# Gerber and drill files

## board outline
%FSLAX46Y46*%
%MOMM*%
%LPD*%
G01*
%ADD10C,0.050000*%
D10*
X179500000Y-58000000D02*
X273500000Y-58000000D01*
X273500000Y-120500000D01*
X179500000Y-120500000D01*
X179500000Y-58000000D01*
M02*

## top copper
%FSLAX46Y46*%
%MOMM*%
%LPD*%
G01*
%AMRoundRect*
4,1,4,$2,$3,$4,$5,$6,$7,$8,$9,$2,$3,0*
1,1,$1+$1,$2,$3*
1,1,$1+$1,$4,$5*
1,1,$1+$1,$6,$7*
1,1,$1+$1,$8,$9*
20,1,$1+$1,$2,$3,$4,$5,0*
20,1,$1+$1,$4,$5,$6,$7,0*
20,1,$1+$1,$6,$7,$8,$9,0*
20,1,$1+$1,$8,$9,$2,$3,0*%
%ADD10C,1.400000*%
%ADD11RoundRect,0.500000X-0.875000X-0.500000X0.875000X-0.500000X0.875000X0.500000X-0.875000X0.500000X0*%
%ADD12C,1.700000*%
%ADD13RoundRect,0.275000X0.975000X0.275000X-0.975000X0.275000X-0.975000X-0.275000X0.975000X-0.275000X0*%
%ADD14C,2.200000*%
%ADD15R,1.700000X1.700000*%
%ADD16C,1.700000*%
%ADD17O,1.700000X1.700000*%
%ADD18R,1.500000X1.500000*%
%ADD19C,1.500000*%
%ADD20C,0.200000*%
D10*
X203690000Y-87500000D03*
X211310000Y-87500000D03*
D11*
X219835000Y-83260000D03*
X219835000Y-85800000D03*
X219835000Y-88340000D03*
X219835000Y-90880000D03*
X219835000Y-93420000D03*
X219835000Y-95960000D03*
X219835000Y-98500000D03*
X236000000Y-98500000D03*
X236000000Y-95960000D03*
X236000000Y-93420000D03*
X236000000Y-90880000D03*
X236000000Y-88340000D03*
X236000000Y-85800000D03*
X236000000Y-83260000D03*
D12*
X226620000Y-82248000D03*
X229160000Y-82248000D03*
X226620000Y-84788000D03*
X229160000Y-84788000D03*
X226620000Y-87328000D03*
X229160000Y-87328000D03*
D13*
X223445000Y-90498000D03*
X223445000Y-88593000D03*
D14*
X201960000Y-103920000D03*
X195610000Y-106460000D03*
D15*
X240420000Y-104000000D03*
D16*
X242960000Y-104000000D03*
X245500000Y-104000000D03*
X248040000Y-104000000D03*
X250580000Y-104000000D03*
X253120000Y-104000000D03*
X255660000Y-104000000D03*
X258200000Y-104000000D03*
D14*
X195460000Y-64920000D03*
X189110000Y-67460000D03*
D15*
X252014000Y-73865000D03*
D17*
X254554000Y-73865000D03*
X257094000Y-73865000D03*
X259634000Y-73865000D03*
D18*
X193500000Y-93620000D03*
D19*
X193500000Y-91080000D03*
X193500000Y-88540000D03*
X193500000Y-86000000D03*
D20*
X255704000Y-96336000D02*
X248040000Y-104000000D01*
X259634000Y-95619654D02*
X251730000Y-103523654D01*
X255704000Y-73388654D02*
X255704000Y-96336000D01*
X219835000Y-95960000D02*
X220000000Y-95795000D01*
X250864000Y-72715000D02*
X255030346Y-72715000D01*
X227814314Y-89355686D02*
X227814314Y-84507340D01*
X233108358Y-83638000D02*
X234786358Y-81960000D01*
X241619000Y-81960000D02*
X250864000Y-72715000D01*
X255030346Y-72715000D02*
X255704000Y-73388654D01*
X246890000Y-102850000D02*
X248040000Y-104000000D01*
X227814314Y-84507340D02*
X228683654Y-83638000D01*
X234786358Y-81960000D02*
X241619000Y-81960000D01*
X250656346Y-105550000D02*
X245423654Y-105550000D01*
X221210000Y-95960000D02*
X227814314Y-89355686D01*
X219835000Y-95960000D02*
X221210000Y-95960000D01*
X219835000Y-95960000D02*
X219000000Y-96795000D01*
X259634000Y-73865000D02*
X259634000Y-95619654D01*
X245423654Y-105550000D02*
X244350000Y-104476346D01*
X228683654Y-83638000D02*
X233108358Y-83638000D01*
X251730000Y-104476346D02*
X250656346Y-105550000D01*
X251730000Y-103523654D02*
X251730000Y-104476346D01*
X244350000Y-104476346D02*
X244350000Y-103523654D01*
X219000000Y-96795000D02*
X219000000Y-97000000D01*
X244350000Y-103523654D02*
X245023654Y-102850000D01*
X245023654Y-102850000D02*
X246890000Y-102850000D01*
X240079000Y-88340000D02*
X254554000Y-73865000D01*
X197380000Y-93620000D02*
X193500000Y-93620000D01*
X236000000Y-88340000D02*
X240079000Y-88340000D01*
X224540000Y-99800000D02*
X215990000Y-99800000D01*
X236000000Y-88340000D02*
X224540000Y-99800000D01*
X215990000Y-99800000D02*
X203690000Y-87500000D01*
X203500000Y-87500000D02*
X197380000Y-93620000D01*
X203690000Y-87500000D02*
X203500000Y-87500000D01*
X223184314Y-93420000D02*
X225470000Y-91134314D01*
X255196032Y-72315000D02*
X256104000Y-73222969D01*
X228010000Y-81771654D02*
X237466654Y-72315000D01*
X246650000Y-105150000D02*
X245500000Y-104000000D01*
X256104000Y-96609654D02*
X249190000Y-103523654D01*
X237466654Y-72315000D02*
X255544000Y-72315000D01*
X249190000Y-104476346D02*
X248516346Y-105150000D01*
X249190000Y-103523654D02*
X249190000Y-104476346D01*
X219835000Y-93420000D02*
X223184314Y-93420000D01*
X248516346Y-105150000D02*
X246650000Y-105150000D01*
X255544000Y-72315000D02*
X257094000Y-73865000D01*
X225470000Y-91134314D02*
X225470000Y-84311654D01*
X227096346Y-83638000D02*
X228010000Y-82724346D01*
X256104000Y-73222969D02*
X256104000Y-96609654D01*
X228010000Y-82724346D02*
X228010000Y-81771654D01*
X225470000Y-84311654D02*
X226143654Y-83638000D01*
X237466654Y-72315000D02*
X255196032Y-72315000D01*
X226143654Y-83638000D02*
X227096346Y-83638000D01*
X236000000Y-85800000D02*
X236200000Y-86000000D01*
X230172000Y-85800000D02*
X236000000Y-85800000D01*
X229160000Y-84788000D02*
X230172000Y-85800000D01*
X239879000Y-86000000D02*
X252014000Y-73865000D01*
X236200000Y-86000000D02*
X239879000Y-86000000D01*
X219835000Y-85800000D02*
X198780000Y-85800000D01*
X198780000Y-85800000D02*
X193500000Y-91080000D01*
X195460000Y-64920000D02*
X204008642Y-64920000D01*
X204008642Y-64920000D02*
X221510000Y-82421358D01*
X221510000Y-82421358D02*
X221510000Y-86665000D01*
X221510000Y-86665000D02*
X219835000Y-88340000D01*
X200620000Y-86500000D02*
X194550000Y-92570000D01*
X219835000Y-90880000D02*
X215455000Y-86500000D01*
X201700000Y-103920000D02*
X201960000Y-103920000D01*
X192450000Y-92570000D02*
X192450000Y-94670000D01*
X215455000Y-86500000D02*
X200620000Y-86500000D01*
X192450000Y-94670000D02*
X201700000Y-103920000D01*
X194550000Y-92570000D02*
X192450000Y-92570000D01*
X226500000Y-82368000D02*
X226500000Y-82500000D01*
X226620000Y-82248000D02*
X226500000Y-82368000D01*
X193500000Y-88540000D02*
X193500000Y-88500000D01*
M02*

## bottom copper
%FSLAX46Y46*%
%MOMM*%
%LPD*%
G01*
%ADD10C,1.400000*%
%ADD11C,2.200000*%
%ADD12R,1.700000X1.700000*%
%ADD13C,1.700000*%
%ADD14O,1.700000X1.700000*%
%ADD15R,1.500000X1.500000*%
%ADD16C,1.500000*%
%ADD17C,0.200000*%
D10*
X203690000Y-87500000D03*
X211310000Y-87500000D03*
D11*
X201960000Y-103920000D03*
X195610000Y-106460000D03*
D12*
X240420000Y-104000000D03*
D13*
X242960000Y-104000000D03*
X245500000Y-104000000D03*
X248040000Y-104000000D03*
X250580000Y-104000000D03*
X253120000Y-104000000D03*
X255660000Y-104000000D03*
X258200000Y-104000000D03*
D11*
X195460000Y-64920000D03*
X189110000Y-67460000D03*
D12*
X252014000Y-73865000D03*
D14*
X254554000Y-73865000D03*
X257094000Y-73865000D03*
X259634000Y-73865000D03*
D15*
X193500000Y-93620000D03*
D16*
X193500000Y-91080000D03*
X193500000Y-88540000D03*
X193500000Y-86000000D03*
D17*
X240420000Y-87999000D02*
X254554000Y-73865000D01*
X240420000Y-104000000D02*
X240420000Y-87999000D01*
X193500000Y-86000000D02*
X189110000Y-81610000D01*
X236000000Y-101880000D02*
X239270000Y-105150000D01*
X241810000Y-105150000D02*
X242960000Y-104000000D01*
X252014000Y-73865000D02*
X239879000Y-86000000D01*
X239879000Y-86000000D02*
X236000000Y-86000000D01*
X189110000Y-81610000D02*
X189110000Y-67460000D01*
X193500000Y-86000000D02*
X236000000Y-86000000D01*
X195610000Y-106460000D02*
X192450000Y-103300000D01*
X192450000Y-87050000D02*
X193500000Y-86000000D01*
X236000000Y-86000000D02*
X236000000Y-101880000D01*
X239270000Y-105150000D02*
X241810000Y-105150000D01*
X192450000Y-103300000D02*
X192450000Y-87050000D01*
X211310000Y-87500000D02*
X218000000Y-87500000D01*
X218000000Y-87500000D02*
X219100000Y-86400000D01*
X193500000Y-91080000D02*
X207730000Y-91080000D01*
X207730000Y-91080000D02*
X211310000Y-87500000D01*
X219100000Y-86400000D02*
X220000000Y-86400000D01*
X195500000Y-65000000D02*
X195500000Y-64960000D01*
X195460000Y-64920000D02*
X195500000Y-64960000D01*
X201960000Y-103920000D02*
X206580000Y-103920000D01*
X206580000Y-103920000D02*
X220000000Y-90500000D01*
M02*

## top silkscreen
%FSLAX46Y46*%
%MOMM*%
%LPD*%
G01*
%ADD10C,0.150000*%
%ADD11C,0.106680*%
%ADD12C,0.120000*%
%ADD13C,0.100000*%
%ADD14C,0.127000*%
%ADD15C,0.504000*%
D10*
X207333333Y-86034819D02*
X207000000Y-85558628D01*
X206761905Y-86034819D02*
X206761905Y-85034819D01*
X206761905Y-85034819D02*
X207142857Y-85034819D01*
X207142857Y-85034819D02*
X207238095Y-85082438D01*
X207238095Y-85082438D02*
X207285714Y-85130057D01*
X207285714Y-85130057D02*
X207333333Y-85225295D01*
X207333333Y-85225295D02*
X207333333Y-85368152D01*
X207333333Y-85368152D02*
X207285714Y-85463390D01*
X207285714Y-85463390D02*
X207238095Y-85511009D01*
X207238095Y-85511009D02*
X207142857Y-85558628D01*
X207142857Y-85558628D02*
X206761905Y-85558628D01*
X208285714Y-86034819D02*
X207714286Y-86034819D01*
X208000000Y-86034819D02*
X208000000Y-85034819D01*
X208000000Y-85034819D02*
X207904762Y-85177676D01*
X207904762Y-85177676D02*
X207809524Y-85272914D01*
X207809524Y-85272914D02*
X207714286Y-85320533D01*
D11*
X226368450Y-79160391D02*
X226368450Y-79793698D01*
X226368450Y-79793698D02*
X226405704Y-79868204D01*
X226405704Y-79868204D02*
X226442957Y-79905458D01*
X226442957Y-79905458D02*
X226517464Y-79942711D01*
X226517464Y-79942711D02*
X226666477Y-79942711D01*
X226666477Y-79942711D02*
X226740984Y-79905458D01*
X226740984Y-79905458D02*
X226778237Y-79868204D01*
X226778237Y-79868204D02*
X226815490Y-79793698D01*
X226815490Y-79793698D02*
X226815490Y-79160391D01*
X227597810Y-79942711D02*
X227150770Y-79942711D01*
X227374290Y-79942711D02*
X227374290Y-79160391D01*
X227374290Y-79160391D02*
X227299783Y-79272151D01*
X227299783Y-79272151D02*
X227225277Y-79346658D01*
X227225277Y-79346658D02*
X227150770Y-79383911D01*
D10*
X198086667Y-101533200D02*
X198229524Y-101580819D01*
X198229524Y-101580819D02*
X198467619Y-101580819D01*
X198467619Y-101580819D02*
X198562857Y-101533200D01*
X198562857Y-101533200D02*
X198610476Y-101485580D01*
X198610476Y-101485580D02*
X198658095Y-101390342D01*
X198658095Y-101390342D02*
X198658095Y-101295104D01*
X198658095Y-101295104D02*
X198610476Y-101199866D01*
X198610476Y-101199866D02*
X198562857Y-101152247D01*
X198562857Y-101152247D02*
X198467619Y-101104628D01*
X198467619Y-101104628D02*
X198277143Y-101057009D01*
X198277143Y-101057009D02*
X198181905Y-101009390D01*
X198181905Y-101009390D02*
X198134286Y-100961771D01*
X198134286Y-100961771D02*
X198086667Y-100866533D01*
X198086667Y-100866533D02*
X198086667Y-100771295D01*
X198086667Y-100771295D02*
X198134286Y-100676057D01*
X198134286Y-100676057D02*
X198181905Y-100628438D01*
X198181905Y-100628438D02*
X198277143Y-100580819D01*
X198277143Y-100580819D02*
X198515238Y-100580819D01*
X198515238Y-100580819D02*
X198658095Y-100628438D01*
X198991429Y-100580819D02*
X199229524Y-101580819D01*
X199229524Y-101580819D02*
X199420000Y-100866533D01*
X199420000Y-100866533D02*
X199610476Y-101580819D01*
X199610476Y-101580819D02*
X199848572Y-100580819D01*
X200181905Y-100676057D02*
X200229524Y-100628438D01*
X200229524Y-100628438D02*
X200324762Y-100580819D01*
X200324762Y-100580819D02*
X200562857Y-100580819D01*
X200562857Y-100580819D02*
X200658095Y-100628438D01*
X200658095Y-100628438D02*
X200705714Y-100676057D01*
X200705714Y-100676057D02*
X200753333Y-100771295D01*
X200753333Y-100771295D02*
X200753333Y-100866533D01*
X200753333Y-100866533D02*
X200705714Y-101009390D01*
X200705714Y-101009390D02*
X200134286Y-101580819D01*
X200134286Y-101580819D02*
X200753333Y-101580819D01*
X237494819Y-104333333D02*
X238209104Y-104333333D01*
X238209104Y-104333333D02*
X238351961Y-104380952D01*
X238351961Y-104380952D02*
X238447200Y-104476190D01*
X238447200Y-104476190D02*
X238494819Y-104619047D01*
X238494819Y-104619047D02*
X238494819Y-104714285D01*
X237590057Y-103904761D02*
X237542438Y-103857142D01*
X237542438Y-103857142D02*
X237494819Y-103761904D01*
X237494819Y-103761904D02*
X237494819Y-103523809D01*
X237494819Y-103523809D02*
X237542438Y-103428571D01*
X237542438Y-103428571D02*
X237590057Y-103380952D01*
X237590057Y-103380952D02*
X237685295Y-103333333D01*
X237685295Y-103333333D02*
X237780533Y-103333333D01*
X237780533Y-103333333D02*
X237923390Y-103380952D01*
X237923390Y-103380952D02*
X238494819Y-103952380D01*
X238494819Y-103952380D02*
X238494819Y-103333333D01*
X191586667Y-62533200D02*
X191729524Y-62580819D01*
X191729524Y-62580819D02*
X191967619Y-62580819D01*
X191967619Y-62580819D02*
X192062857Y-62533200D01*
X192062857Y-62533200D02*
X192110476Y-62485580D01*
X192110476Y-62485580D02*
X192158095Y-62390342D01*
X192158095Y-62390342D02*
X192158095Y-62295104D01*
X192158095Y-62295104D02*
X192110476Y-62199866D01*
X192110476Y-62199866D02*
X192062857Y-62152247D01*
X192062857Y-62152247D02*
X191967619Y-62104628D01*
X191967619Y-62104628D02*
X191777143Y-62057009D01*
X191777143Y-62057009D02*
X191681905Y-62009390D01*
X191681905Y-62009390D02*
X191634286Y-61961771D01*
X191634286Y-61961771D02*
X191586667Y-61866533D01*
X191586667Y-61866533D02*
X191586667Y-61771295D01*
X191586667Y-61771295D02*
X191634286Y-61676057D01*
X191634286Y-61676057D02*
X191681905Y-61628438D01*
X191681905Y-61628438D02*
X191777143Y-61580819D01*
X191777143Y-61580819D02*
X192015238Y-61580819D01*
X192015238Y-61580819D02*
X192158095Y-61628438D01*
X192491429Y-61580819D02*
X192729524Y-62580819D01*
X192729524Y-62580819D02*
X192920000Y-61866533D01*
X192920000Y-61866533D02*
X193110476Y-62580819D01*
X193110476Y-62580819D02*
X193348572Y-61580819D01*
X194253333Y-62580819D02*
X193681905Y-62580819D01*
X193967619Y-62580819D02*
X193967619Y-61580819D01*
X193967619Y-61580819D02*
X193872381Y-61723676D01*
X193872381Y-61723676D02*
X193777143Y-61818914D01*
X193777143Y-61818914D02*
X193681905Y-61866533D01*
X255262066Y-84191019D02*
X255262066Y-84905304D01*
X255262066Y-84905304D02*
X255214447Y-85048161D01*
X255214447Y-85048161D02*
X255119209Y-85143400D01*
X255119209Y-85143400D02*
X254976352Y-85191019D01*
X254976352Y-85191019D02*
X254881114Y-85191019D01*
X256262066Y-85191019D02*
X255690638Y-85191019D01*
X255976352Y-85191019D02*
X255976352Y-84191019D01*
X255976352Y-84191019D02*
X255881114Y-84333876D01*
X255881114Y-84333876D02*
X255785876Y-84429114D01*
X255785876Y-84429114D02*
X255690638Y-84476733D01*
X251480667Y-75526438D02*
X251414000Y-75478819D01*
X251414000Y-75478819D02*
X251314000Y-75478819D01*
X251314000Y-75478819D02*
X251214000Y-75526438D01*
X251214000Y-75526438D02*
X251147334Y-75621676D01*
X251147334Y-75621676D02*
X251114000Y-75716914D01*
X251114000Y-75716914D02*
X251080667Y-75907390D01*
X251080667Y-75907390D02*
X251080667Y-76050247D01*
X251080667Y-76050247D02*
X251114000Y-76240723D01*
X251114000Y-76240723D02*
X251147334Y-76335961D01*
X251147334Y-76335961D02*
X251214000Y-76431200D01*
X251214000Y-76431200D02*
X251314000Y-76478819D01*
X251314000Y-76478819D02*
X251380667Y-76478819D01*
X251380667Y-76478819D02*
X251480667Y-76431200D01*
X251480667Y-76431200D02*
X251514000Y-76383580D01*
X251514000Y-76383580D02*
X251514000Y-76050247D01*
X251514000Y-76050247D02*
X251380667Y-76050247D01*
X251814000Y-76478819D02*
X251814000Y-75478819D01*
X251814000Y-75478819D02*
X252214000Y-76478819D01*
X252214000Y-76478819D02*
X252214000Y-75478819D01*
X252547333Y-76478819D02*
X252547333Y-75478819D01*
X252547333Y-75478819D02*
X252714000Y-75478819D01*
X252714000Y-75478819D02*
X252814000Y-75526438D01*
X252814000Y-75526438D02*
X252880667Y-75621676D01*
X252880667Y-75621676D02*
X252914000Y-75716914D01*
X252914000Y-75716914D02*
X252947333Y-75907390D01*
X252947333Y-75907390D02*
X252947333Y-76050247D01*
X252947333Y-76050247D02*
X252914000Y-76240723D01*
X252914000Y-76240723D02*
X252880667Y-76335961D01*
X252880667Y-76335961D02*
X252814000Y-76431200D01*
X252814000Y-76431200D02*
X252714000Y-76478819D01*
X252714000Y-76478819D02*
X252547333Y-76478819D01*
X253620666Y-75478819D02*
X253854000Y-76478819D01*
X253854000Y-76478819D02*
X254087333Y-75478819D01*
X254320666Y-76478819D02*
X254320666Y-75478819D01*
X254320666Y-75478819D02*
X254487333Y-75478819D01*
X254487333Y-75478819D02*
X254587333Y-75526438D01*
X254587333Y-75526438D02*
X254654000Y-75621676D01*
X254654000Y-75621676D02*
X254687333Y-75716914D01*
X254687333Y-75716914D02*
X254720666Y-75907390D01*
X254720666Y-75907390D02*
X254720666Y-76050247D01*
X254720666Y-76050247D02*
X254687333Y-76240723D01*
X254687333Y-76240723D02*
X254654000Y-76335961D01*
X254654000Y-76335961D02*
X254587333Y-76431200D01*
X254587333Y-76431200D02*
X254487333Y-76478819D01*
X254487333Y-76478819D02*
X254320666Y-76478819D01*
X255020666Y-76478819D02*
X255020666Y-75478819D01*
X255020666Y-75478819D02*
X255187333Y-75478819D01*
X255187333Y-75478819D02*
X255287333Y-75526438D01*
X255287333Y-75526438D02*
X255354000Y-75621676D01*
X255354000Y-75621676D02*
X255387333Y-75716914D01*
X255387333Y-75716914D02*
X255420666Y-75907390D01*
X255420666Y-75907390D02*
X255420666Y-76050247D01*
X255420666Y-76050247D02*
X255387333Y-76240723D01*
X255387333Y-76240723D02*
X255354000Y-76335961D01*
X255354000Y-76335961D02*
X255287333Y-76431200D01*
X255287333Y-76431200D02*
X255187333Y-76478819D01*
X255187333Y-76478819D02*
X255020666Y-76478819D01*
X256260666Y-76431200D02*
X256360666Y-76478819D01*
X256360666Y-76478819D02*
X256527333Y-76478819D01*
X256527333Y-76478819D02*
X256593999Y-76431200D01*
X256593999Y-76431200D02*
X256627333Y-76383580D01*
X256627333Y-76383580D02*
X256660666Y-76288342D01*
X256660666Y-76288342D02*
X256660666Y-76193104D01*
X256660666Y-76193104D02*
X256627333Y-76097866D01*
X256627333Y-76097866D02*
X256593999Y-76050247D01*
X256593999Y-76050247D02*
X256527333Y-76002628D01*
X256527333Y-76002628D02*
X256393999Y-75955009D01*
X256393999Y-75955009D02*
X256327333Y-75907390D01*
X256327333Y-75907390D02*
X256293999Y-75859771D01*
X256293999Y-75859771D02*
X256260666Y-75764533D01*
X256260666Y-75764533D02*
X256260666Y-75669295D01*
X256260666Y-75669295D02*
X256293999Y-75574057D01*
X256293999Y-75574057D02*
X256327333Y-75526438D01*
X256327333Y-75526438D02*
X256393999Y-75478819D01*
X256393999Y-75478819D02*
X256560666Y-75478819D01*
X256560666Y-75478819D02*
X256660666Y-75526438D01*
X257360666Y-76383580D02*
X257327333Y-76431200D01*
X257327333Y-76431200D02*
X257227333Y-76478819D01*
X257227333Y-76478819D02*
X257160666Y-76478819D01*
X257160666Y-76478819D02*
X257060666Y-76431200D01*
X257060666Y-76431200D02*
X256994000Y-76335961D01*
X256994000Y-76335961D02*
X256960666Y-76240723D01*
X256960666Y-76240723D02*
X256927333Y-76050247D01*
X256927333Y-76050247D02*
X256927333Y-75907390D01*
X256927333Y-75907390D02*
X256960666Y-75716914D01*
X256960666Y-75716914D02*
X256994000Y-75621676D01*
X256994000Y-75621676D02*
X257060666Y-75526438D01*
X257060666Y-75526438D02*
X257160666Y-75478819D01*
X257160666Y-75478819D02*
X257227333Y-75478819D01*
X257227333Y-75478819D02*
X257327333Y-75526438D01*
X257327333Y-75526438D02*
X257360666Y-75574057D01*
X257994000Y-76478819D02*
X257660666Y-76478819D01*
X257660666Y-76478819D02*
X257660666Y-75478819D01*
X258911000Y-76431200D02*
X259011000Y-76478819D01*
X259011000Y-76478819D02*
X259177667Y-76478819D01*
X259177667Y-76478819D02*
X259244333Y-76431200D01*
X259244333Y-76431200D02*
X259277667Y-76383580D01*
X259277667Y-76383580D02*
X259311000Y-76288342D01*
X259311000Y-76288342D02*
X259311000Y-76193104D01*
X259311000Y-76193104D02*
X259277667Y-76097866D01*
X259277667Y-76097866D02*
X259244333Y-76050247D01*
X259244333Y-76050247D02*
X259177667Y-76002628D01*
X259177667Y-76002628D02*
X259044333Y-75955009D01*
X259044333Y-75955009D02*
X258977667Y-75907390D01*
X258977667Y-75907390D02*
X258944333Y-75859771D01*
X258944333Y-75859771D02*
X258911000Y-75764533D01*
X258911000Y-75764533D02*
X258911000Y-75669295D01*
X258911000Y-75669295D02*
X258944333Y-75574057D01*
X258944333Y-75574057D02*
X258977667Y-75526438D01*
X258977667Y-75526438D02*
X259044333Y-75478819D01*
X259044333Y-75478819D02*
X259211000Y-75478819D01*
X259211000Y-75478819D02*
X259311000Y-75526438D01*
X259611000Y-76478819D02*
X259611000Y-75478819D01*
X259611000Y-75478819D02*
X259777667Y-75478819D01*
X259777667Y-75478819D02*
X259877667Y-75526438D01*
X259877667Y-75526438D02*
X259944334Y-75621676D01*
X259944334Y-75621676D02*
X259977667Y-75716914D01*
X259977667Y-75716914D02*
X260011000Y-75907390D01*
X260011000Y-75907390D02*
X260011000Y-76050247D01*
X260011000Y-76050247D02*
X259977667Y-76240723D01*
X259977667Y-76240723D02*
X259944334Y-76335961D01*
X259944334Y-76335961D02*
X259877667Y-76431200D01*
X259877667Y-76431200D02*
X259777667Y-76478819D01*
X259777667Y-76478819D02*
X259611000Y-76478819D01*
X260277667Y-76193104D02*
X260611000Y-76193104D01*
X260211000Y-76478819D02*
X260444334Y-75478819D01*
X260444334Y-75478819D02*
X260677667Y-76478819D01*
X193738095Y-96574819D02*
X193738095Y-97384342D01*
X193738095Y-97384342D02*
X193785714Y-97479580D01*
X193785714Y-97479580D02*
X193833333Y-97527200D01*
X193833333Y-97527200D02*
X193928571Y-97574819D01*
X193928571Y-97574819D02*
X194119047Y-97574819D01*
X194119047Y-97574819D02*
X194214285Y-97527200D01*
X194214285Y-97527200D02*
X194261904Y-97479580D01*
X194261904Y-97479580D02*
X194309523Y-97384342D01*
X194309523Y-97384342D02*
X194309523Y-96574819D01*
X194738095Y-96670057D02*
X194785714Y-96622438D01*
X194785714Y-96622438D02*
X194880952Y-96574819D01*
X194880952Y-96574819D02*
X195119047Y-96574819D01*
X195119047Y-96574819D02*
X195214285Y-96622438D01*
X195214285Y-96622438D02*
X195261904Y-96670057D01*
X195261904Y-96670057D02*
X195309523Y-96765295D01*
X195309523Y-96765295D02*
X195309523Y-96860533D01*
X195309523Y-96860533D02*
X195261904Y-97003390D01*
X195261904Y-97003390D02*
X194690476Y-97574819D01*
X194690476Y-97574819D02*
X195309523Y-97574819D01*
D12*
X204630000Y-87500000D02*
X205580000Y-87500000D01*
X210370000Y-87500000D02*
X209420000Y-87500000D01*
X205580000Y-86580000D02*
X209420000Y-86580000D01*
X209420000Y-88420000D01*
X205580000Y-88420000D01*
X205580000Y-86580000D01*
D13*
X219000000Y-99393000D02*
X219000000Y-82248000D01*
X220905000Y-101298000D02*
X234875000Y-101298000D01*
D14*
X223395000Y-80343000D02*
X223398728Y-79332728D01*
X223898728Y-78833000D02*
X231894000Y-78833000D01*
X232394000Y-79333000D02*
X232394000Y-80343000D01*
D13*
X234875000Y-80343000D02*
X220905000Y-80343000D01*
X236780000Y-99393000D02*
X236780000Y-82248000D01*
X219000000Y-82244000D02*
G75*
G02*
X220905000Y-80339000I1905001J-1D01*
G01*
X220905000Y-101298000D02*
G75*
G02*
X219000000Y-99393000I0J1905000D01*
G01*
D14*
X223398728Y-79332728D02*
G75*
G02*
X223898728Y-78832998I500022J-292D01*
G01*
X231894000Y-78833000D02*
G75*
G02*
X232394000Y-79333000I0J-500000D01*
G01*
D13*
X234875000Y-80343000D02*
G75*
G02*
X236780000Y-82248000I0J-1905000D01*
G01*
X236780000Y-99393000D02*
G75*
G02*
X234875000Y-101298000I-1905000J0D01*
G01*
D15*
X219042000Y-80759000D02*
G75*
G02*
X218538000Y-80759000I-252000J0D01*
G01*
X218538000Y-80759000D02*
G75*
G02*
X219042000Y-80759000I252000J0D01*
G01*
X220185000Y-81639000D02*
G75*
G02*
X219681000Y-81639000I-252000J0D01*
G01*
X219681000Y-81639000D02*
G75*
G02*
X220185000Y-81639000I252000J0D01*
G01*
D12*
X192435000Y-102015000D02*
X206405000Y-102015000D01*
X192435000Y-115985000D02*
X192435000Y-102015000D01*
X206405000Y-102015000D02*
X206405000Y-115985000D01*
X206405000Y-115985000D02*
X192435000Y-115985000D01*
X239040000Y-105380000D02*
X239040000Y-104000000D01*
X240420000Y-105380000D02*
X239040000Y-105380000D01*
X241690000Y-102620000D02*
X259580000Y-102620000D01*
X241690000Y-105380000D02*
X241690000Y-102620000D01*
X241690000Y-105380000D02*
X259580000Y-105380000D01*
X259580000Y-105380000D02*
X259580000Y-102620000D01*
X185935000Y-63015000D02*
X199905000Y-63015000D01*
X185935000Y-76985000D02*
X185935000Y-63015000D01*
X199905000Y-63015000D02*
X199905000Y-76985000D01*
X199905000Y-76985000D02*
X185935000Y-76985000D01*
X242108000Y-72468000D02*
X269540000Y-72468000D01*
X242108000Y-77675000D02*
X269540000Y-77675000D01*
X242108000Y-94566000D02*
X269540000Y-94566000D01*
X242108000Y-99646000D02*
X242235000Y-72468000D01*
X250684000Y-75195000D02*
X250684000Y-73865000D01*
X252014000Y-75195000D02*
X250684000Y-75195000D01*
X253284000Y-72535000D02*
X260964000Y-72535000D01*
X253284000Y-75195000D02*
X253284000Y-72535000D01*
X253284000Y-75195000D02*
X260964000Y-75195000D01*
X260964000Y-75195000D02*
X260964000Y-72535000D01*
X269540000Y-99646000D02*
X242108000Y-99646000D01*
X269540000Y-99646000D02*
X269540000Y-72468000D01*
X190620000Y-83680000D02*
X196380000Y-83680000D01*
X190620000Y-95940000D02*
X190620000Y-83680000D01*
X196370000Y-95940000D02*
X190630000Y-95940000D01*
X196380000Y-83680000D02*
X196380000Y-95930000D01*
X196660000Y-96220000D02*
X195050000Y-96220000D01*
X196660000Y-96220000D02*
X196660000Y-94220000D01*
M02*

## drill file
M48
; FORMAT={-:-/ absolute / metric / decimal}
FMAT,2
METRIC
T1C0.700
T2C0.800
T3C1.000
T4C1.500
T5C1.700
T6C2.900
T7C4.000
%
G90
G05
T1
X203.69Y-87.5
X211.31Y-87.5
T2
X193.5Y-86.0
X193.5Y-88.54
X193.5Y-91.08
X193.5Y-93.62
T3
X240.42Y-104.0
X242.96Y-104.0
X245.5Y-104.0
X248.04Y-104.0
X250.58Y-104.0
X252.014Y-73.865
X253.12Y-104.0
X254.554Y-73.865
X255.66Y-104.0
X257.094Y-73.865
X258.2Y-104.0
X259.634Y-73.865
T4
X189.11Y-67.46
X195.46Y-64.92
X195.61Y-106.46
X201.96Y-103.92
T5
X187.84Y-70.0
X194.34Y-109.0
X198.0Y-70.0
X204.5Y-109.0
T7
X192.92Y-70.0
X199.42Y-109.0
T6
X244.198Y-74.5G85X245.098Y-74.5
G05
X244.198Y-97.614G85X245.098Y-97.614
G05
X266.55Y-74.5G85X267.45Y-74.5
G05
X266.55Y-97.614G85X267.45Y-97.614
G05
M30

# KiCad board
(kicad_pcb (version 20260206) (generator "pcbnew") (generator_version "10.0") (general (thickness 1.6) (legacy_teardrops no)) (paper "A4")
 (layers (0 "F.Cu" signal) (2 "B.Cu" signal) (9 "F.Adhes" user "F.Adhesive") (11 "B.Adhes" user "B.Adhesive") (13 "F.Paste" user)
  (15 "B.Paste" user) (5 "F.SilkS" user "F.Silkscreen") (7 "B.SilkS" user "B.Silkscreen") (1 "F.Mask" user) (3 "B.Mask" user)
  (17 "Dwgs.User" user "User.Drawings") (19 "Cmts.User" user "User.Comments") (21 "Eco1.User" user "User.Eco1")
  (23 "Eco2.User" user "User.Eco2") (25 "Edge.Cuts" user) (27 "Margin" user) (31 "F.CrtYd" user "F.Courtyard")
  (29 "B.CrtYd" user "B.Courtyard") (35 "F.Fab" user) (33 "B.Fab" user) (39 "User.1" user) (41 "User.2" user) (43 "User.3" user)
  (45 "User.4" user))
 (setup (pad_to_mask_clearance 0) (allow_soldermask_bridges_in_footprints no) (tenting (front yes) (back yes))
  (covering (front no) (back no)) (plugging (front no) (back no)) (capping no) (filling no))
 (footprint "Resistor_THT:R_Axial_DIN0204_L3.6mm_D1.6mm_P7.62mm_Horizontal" (layer "F.Cu") (at 203.69 87.5)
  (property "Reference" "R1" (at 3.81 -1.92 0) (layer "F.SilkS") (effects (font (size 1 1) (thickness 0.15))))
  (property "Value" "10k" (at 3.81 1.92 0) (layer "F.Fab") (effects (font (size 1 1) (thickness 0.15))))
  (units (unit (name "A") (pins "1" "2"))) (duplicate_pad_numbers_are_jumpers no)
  (fp_line (start 0.94 0) (end 1.89 0) (stroke (width 0.12) (type solid)) (layer "F.SilkS"))
  (fp_line (start 6.68 0) (end 5.73 0) (stroke (width 0.12) (type solid)) (layer "F.SilkS"))
  (fp_rect (start 1.89 -0.92) (end 5.73 0.92) (stroke (width 0.12) (type solid)) (fill no) (layer "F.SilkS"))
  (pad "1" thru_hole circle (at 0 0) (size 1.4 1.4) (drill 0.7) (layers "*.Cu" "*.Mask") (remove_unused_layers no) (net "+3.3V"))
  (pad "2" thru_hole circle (at 7.62 0) (size 1.4 1.4) (drill 0.7) (layers "*.Cu" "*.Mask") (remove_unused_layers no) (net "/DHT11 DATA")))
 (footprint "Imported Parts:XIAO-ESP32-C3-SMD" (layer "F.Cu") (at 219 101.38)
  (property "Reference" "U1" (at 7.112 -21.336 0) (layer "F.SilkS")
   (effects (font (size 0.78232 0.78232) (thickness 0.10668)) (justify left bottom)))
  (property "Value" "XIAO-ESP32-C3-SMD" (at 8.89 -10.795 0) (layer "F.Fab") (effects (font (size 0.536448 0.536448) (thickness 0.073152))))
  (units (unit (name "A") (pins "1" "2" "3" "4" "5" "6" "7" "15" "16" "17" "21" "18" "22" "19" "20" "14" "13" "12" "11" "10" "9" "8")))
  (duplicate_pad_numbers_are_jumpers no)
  (fp_line (start 0 -1.987) (end 0 -19.132) (stroke (width 0.1) (type solid)) (layer "F.SilkS"))
  (fp_line (start 1.905 -0.082) (end 15.875 -0.082) (stroke (width 0.1) (type solid)) (layer "F.SilkS"))
  (fp_line (start 4.395 -21.037) (end 4.398728 -22.047272) (stroke (width 0.127) (type solid)) (layer "F.SilkS"))
  (fp_line (start 4.898728 -22.547) (end 12.894 -22.547) (stroke (width 0.127) (type solid)) (layer "F.SilkS"))
  (fp_line (start 13.394 -22.047) (end 13.394 -21.037) (stroke (width 0.127) (type solid)) (layer "F.SilkS"))
  (fp_line (start 15.875 -21.037) (end 1.905 -21.037) (stroke (width 0.1) (type solid)) (layer "F.SilkS"))
  (fp_line (start 17.78 -1.987) (end 17.78 -19.132) (stroke (width 0.1) (type solid)) (layer "F.SilkS"))
  (fp_arc (start 0 -19.136) (mid 0.557962 -20.483038) (end 1.905 -21.041) (stroke (width 0.1) (type solid)) (layer "F.SilkS"))
  (fp_arc (start 1.905 -0.082) (mid 0.557962 -0.639962) (end 0 -1.987) (stroke (width 0.1) (type solid)) (layer "F.SilkS"))
  (fp_arc (start 4.398728 -22.047272) (mid 4.545272 -22.40064) (end 4.898728 -22.547) (stroke (width 0.127) (type default))
   (layer "F.SilkS"))
  (fp_arc (start 12.894 -22.547) (mid 13.247553 -22.400553) (end 13.394 -22.047) (stroke (width 0.127) (type default)) (layer "F.SilkS"))
  (fp_arc (start 15.875 -21.037) (mid 17.222038 -20.479038) (end 17.78 -19.132) (stroke (width 0.1) (type solid)) (layer "F.SilkS"))
  (fp_arc (start 17.78 -1.987) (mid 17.222038 -0.639962) (end 15.875 -0.082) (stroke (width 0.1) (type solid)) (layer "F.SilkS"))
  (fp_circle (center -0.21 -20.621) (end -0.21 -20.875) (stroke (width 0.5) (type solid)) (fill yes) (layer "F.SilkS"))
  (fp_circle (center 0.933 -19.741) (end 0.933 -19.995) (stroke (width 0.5) (type solid)) (fill yes) (layer "F.SilkS"))
  (pad "1" smd roundrect (at 0.835 -18.12) (size 2.75 2) (layers "F.Cu" "F.Mask" "F.Paste") (roundrect_rratio 0.25)
   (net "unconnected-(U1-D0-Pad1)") (solder_mask_margin 0.0508) (thermal_bridge_angle 45))
  (pad "2" smd roundrect (at 0.835 -15.58) (size 2.75 2) (layers "F.Cu" "F.Mask" "F.Paste") (roundrect_rratio 0.25) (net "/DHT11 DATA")
   (solder_mask_margin 0.0508) (thermal_bridge_angle 45))
  (pad "3" smd roundrect (at 0.835 -13.04) (size 2.75 2) (layers "F.Cu" "F.Mask" "F.Paste") (roundrect_rratio 0.25) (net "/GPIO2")
   (solder_mask_margin 0.0508) (thermal_bridge_angle 45))
  (pad "4" smd roundrect (at 0.835 -10.5) (size 2.75 2) (layers "F.Cu" "F.Mask" "F.Paste") (roundrect_rratio 0.25) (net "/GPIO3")
   (solder_mask_margin 0.0508) (thermal_bridge_angle 45))
  (pad "5" smd roundrect (at 0.835 -7.96) (size 2.75 2) (layers "F.Cu" "F.Mask" "F.Paste") (roundrect_rratio 0.25) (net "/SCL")
   (solder_mask_margin 0.0508) (thermal_bridge_angle 45))
  (pad "6" smd roundrect (at 0.835 -5.42) (size 2.75 2) (layers "F.Cu" "F.Mask" "F.Paste") (roundrect_rratio 0.25) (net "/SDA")
   (solder_mask_margin 0.0508) (thermal_bridge_angle 45))
  (pad "7" smd roundrect (at 0.835 -2.88) (size 2.75 2) (layers "F.Cu" "F.Mask" "F.Paste") (roundrect_rratio 0.25)
   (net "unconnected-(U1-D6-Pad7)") (solder_mask_margin 0.0508) (thermal_bridge_angle 45))
  (pad "8" smd roundrect (at 17 -2.88) (size 2.75 2) (layers "F.Cu" "F.Mask" "F.Paste") (roundrect_rratio 0.25)
   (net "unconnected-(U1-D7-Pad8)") (solder_mask_margin 0.0508) (thermal_bridge_angle 45))
  (pad "9" smd roundrect (at 17 -5.42) (size 2.75 2) (layers "F.Cu" "F.Mask" "F.Paste") (roundrect_rratio 0.25)
   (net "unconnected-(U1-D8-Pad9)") (solder_mask_margin 0.0508) (thermal_bridge_angle 45))
  (pad "10" smd roundrect (at 17 -7.96) (size 2.75 2) (layers "F.Cu" "F.Mask" "F.Paste") (roundrect_rratio 0.25)
   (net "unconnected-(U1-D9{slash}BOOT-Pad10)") (solder_mask_margin 0.0508) (thermal_bridge_angle 45))
  (pad "11" smd roundrect (at 17 -10.5) (size 2.75 2) (layers "F.Cu" "F.Mask" "F.Paste") (roundrect_rratio 0.25)
   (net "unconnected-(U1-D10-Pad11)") (solder_mask_margin 0.0508) (thermal_bridge_angle 45))
  (pad "12" smd roundrect (at 17 -13.04) (size 2.75 2) (layers "F.Cu" "F.Mask" "F.Paste") (roundrect_rratio 0.25) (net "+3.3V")
   (solder_mask_margin 0.0508) (thermal_bridge_angle 45))
  (pad "13" smd roundrect (at 17 -15.58) (size 2.75 2) (layers "F.Cu" "F.Mask" "F.Paste") (roundrect_rratio 0.25) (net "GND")
   (solder_mask_margin 0.0508) (thermal_bridge_angle 45))
  (pad "14" smd roundrect (at 17 -18.12) (size 2.75 2) (layers "F.Cu" "F.Mask" "F.Paste") (roundrect_rratio 0.25) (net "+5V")
   (solder_mask_margin 0.0508) (thermal_bridge_angle 45))
  (pad "15" smd circle (at 7.62 -19.132) (size 1.7 1.7) (layers "F.Cu" "F.Mask" "F.Paste") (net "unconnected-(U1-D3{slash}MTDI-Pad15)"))
  (pad "16" smd circle (at 10.16 -19.132) (size 1.7 1.7) (layers "F.Cu" "F.Mask" "F.Paste") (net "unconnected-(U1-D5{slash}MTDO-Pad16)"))
  (pad "17" smd circle (at 7.62 -16.592) (size 1.7 1.7) (layers "F.Cu" "F.Mask" "F.Paste") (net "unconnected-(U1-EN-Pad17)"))
  (pad "18" smd circle (at 10.16 -16.592) (size 1.7 1.7) (layers "F.Cu" "F.Mask" "F.Paste") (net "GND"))
  (pad "19" smd circle (at 7.62 -14.052) (size 1.7 1.7) (layers "F.Cu" "F.Mask" "F.Paste") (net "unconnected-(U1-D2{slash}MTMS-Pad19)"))
  (pad "20" smd circle (at 10.16 -14.052) (size 1.7 1.7) (layers "F.Cu" "F.Mask" "F.Paste") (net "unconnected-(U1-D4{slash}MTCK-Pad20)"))
  (pad "21" smd roundrect (at 4.445 -10.882 180) (size 2.5 1.1) (layers "F.Cu" "F.Mask" "F.Paste") (roundrect_rratio 0.25)
   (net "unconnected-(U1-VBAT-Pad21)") (thermal_bridge_angle 45))
  (pad "22" smd roundrect (at 4.445 -12.787 180) (size 2.5 1.1) (layers "F.Cu" "F.Mask" "F.Paste") (roundrect_rratio 0.25)
   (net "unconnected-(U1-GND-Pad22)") (thermal_bridge_angle 45)))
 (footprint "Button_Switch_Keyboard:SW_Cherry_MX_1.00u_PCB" (layer "F.Cu") (at 201.96 103.92)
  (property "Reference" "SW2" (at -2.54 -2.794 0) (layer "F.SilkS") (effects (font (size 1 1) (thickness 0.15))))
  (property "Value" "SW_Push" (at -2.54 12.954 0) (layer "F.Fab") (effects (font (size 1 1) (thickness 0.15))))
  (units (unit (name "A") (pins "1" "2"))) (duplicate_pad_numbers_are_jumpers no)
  (fp_line (start -9.525 -1.905) (end 4.445 -1.905) (stroke (width 0.12) (type solid)) (layer "F.SilkS"))
  (fp_line (start -9.525 12.065) (end -9.525 -1.905) (stroke (width 0.12) (type solid)) (layer "F.SilkS"))
  (fp_line (start 4.445 -1.905) (end 4.445 12.065) (stroke (width 0.12) (type solid)) (layer "F.SilkS"))
  (fp_line (start 4.445 12.065) (end -9.525 12.065) (stroke (width 0.12) (type solid)) (layer "F.SilkS"))
  (pad "" np_thru_hole circle (at -7.62 5.08) (size 1.7 1.7) (drill 1.7) (layers "*.Cu" "*.Mask"))
  (pad "" np_thru_hole circle (at -2.54 5.08) (size 4 4) (drill 4) (layers "*.Cu" "*.Mask"))
  (pad "" np_thru_hole circle (at 2.54 5.08) (size 1.7 1.7) (drill 1.7) (layers "*.Cu" "*.Mask"))
  (pad "1" thru_hole circle (at 0 0) (size 2.2 2.2) (drill 1.5) (layers "*.Cu" "*.Mask") (remove_unused_layers no) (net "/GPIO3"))
  (pad "2" thru_hole circle (at -6.35 2.54) (size 2.2 2.2) (drill 1.5) (layers "*.Cu" "*.Mask") (remove_unused_layers no) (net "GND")))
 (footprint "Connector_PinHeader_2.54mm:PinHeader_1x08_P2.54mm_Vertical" (layer "F.Cu") (at 240.42 104 90)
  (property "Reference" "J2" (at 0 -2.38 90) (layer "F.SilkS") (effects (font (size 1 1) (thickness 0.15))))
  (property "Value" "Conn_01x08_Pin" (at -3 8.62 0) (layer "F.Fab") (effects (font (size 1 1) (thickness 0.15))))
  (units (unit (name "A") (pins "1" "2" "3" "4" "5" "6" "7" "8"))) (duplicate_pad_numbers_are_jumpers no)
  (fp_line (start -1.38 -1.38) (end 0 -1.38) (stroke (width 0.12) (type solid)) (layer "F.SilkS"))
  (fp_line (start -1.38 0) (end -1.38 -1.38) (stroke (width 0.12) (type solid)) (layer "F.SilkS"))
  (fp_line (start 1.38 1.27) (end 1.38 19.16) (stroke (width 0.12) (type solid)) (layer "F.SilkS"))
  (fp_line (start -1.38 1.27) (end 1.38 1.27) (stroke (width 0.12) (type solid)) (layer "F.SilkS"))
  (fp_line (start -1.38 1.27) (end -1.38 19.16) (stroke (width 0.12) (type solid)) (layer "F.SilkS"))
  (fp_line (start -1.38 19.16) (end 1.38 19.16) (stroke (width 0.12) (type solid)) (layer "F.SilkS"))
  (pad "1" thru_hole rect (at 0 0 90) (size 1.7 1.7) (drill 1) (layers "*.Cu" "*.Mask") (remove_unused_layers no) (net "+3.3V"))
  (pad "2" thru_hole circle (at 0 2.54 90) (size 1.7 1.7) (drill 1) (layers "*.Cu" "*.Mask") (remove_unused_layers no) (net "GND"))
  (pad "3" thru_hole circle (at 0 5.08 90) (size 1.7 1.7) (drill 1) (layers "*.Cu" "*.Mask") (remove_unused_layers no) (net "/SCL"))
  (pad "4" thru_hole circle (at 0 7.62 90) (size 1.7 1.7) (drill 1) (layers "*.Cu" "*.Mask") (remove_unused_layers no) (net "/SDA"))
  (pad "5" thru_hole circle (at 0 10.16 90) (size 1.7 1.7) (drill 1) (layers "*.Cu" "*.Mask") (remove_unused_layers no)
   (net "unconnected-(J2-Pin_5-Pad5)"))
  (pad "6" thru_hole circle (at 0 12.7 90) (size 1.7 1.7) (drill 1) (layers "*.Cu" "*.Mask") (remove_unused_layers no)
   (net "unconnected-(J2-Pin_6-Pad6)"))
  (pad "7" thru_hole circle (at 0 15.24 90) (size 1.7 1.7) (drill 1) (layers "*.Cu" "*.Mask") (remove_unused_layers no)
   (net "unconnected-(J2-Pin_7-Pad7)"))
  (pad "8" thru_hole circle (at 0 17.78 90) (size 1.7 1.7) (drill 1) (layers "*.Cu" "*.Mask") (remove_unused_layers no)
   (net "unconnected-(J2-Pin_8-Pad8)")))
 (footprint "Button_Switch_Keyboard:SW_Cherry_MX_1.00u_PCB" (layer "F.Cu") (at 195.46 64.92)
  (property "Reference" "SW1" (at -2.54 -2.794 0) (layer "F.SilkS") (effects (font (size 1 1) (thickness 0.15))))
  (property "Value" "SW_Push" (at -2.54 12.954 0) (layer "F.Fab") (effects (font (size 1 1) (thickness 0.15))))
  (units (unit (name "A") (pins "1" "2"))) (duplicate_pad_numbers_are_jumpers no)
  (fp_line (start -9.525 -1.905) (end 4.445 -1.905) (stroke (width 0.12) (type solid)) (layer "F.SilkS"))
  (fp_line (start -9.525 12.065) (end -9.525 -1.905) (stroke (width 0.12) (type solid)) (layer "F.SilkS"))
  (fp_line (start 4.445 -1.905) (end 4.445 12.065) (stroke (width 0.12) (type solid)) (layer "F.SilkS"))
  (fp_line (start 4.445 12.065) (end -9.525 12.065) (stroke (width 0.12) (type solid)) (layer "F.SilkS"))
  (pad "" np_thru_hole circle (at -7.62 5.08) (size 1.7 1.7) (drill 1.7) (layers "*.Cu" "*.Mask"))
  (pad "" np_thru_hole circle (at -2.54 5.08) (size 4 4) (drill 4) (layers "*.Cu" "*.Mask"))
  (pad "" np_thru_hole circle (at 2.54 5.08) (size 1.7 1.7) (drill 1.7) (layers "*.Cu" "*.Mask"))
  (pad "1" thru_hole circle (at 0 0) (size 2.2 2.2) (drill 1.5) (layers "*.Cu" "*.Mask") (remove_unused_layers no) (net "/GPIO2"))
  (pad "2" thru_hole circle (at -6.35 2.54) (size 2.2 2.2) (drill 1.5) (layers "*.Cu" "*.Mask") (remove_unused_layers no) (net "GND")))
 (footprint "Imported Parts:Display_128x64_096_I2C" (layer "F.Cu") (at 255.824 73.865)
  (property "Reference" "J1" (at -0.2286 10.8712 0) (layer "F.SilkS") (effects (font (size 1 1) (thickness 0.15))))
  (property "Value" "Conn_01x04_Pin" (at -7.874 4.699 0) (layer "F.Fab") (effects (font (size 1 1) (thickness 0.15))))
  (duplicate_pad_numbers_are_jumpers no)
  (fp_line (start -13.716 -1.397) (end 13.716 -1.397) (stroke (width 0.12) (type solid)) (layer "F.SilkS"))
  (fp_line (start -13.716 3.81) (end 13.716 3.81) (stroke (width 0.12) (type solid)) (layer "F.SilkS"))
  (fp_line (start -13.716 20.701) (end 13.716 20.701) (stroke (width 0.12) (type solid)) (layer "F.SilkS"))
  (fp_line (start -13.716 25.781) (end -13.589 -1.397) (stroke (width 0.12) (type solid)) (layer "F.SilkS"))
  (fp_line (start -5.14 1.33) (end -5.14 0) (stroke (width 0.12) (type solid)) (layer "F.SilkS"))
  (fp_line (start -3.81 1.33) (end -5.14 1.33) (stroke (width 0.12) (type solid)) (layer "F.SilkS"))
  (fp_line (start -2.54 -1.33) (end 5.14 -1.33) (stroke (width 0.12) (type solid)) (layer "F.SilkS"))
  (fp_line (start -2.54 1.33) (end -2.54 -1.33) (stroke (width 0.12) (type solid)) (layer "F.SilkS"))
  (fp_line (start -2.54 1.33) (end 5.14 1.33) (stroke (width 0.12) (type solid)) (layer "F.SilkS"))
  (fp_line (start 5.14 1.33) (end 5.14 -1.33) (stroke (width 0.12) (type solid)) (layer "F.SilkS"))
  (fp_line (start 13.716 25.781) (end -13.716 25.781) (stroke (width 0.12) (type solid)) (layer "F.SilkS"))
  (fp_line (start 13.716 25.781) (end 13.716 -1.397) (stroke (width 0.12) (type solid)) (layer "F.SilkS"))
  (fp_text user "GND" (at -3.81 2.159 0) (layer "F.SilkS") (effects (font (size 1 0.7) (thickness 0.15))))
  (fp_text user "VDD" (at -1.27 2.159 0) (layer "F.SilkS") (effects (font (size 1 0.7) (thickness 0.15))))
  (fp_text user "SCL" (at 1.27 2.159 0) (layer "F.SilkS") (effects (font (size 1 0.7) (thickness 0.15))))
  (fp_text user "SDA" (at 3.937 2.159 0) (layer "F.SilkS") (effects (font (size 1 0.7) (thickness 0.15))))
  (pad "" np_thru_hole oval (at -11.176 0.635) (size 3.8 2.9) (drill oval 3.8 2.9) (layers "*.Cu" "*.Mask"))
  (pad "" np_thru_hole oval (at -11.176 23.749) (size 3.8 2.9) (drill oval 3.8 2.9) (layers "*.Cu" "*.Mask"))
  (pad "" np_thru_hole oval (at 11.176 0.635) (size 3.8 2.9) (drill oval 3.8 2.9) (layers "*.Cu" "*.Mask"))
  (pad "" np_thru_hole oval (at 11.176 23.749) (size 3.8 2.9) (drill oval 3.8 2.9) (layers "*.Cu" "*.Mask"))
  (pad "1" thru_hole rect (at -3.81 0 90) (size 1.7 1.7) (drill 1) (layers "*.Cu" "*.Mask") (remove_unused_layers no) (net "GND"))
  (pad "2" thru_hole oval (at -1.27 0 90) (size 1.7 1.7) (drill 1) (layers "*.Cu" "*.Mask") (remove_unused_layers no) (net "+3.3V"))
  (pad "3" thru_hole oval (at 1.27 0 90) (size 1.7 1.7) (drill 1) (layers "*.Cu" "*.Mask") (remove_unused_layers no) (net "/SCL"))
  (pad "4" thru_hole oval (at 3.81 0 90) (size 1.7 1.7) (drill 1) (layers "*.Cu" "*.Mask") (remove_unused_layers no) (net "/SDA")))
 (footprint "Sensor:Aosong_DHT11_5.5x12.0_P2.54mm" (layer "F.Cu") (at 193.5 93.62 180)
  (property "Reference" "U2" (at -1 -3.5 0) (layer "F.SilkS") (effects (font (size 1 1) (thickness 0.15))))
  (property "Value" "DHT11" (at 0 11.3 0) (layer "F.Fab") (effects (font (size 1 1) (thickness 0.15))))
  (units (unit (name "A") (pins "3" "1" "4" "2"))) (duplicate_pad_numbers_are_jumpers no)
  (fp_line (start 2.88 9.94) (end -2.88 9.94) (stroke (width 0.12) (type solid)) (layer "F.SilkS"))
  (fp_line (start 2.88 -2.32) (end 2.88 9.94) (stroke (width 0.12) (type solid)) (layer "F.SilkS"))
  (fp_line (start -2.87 -2.32) (end 2.87 -2.32) (stroke (width 0.12) (type solid)) (layer "F.SilkS"))
  (fp_line (start -2.88 9.94) (end -2.88 -2.31) (stroke (width 0.12) (type solid)) (layer "F.SilkS"))
  (fp_line (start -3.16 -2.6) (end -1.55 -2.6) (stroke (width 0.12) (type solid)) (layer "F.SilkS"))
  (fp_line (start -3.16 -2.6) (end -3.16 -0.6) (stroke (width 0.12) (type solid)) (layer "F.SilkS"))
  (pad "1" thru_hole rect (at 0 0 180) (size 1.5 1.5) (drill 0.8) (layers "*.Cu" "*.Mask") (remove_unused_layers no) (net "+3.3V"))
  (pad "2" thru_hole circle (at 0 2.54 180) (size 1.5 1.5) (drill 0.8) (layers "*.Cu" "*.Mask") (remove_unused_layers no)
   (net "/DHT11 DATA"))
  (pad "3" thru_hole circle (at 0 5.08 180) (size 1.5 1.5) (drill 0.8) (layers "*.Cu" "*.Mask") (remove_unused_layers no)
   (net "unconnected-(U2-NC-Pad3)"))
  (pad "4" thru_hole circle (at 0 7.62 180) (size 1.5 1.5) (drill 0.8) (layers "*.Cu" "*.Mask") (remove_unused_layers no) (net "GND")))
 (gr_rect (start 179.5 58) (end 273.5 120.5) (stroke (width 0.05) (type default)) (fill no) (layer "Edge.Cuts"))
 (segment (start 255.704 96.336) (end 248.04 104) (width 0.2) (layer "F.Cu") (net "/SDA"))
 (segment (start 259.634 95.619654) (end 251.73 103.523654) (width 0.2) (layer "F.Cu") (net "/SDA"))
 (segment (start 255.704 73.388654) (end 255.704 96.336) (width 0.2) (layer "F.Cu") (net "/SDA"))
 (segment (start 219.835 95.96) (end 220 95.795) (width 0.2) (layer "F.Cu") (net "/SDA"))
 (segment (start 250.864 72.715) (end 255.030346 72.715) (width 0.2) (layer "F.Cu") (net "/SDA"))
 (segment (start 227.814314 89.355686) (end 227.814314 84.50734) (width 0.2) (layer "F.Cu") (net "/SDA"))
 (segment (start 233.108358 83.638) (end 234.786358 81.96) (width 0.2) (layer "F.Cu") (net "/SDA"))
 (segment (start 241.619 81.96) (end 250.864 72.715) (width 0.2) (layer "F.Cu") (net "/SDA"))
 (segment (start 255.030346 72.715) (end 255.704 73.388654) (width 0.2) (layer "F.Cu") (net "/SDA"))
 (segment (start 246.89 102.85) (end 248.04 104) (width 0.2) (layer "F.Cu") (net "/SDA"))
 (segment (start 227.814314 84.50734) (end 228.683654 83.638) (width 0.2) (layer "F.Cu") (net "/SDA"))
 (segment (start 234.786358 81.96) (end 241.619 81.96) (width 0.2) (layer "F.Cu") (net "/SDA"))
 (segment (start 250.656346 105.55) (end 245.423654 105.55) (width 0.2) (layer "F.Cu") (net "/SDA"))
 (segment (start 221.21 95.96) (end 227.814314 89.355686) (width 0.2) (layer "F.Cu") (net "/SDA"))
 (segment (start 219.835 95.96) (end 221.21 95.96) (width 0.2) (layer "F.Cu") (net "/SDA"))
 (segment (start 219.835 95.96) (end 219 96.795) (width 0.2) (layer "F.Cu") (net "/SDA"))
 (segment (start 259.634 73.865) (end 259.634 95.619654) (width 0.2) (layer "F.Cu") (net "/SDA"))
 (segment (start 245.423654 105.55) (end 244.35 104.476346) (width 0.2) (layer "F.Cu") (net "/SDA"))
 (segment (start 228.683654 83.638) (end 233.108358 83.638) (width 0.2) (layer "F.Cu") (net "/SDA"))
 (segment (start 251.73 104.476346) (end 250.656346 105.55) (width 0.2) (layer "F.Cu") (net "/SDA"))
 (segment (start 251.73 103.523654) (end 251.73 104.476346) (width 0.2) (layer "F.Cu") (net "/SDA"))
 (segment (start 244.35 104.476346) (end 244.35 103.523654) (width 0.2) (layer "F.Cu") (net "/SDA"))
 (segment (start 219 96.795) (end 219 97) (width 0.2) (layer "F.Cu") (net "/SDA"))
 (segment (start 244.35 103.523654) (end 245.023654 102.85) (width 0.2) (layer "F.Cu") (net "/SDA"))
 (segment (start 245.023654 102.85) (end 246.89 102.85) (width 0.2) (layer "F.Cu") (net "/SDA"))
 (segment (start 240.079 88.34) (end 254.554 73.865) (width 0.2) (layer "F.Cu") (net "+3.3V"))
 (segment (start 197.38 93.62) (end 193.5 93.62) (width 0.2) (layer "F.Cu") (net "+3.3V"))
 (segment (start 236 88.34) (end 240.079 88.34) (width 0.2) (layer "F.Cu") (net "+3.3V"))
 (segment (start 224.54 99.8) (end 215.99 99.8) (width 0.2) (layer "F.Cu") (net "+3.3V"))
 (segment (start 236 88.34) (end 224.54 99.8) (width 0.2) (layer "F.Cu") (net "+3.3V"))
 (segment (start 215.99 99.8) (end 203.69 87.5) (width 0.2) (layer "F.Cu") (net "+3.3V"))
 (segment (start 203.5 87.5) (end 197.38 93.62) (width 0.2) (layer "F.Cu") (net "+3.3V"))
 (segment (start 203.69 87.5) (end 203.5 87.5) (width 0.2) (layer "F.Cu") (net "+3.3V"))
 (segment (start 240.42 87.999) (end 254.554 73.865) (width 0.2) (layer "B.Cu") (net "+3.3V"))
 (segment (start 240.42 104) (end 240.42 87.999) (width 0.2) (layer "B.Cu") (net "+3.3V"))
 (segment (start 223.184314 93.42) (end 225.47 91.134314) (width 0.2) (layer "F.Cu") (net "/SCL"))
 (segment (start 255.196032 72.315) (end 256.104 73.222969) (width 0.2) (layer "F.Cu") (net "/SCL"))
 (segment (start 228.01 81.771654) (end 237.466654 72.315) (width 0.2) (layer "F.Cu") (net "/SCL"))
 (segment (start 246.65 105.15) (end 245.5 104) (width 0.2) (layer "F.Cu") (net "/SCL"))
 (segment (start 256.104 96.609654) (end 249.19 103.523654) (width 0.2) (layer "F.Cu") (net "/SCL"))
 (segment (start 237.466654 72.315) (end 255.544 72.315) (width 0.2) (layer "F.Cu") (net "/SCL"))
 (segment (start 249.19 104.476346) (end 248.516346 105.15) (width 0.2) (layer "F.Cu") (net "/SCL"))
 (segment (start 249.19 103.523654) (end 249.19 104.476346) (width 0.2) (layer "F.Cu") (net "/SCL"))
 (segment (start 219.835 93.42) (end 223.184314 93.42) (width 0.2) (layer "F.Cu") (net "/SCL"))
 (segment (start 248.516346 105.15) (end 246.65 105.15) (width 0.2) (layer "F.Cu") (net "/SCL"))
 (segment (start 255.544 72.315) (end 257.094 73.865) (width 0.2) (layer "F.Cu") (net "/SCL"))
 (segment (start 225.47 91.134314) (end 225.47 84.311654) (width 0.2) (layer "F.Cu") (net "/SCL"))
 (segment (start 227.096346 83.638) (end 228.01 82.724346) (width 0.2) (layer "F.Cu") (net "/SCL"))
 (segment (start 256.104 73.222969) (end 256.104 96.609654) (width 0.2) (layer "F.Cu") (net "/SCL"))
 (segment (start 228.01 82.724346) (end 228.01 81.771654) (width 0.2) (layer "F.Cu") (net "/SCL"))
 (segment (start 225.47 84.311654) (end 226.143654 83.638) (width 0.2) (layer "F.Cu") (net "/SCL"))
 (segment (start 237.466654 72.315) (end 255.196032 72.315) (width 0.2) (layer "F.Cu") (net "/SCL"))
 (segment (start 226.143654 83.638) (end 227.096346 83.638) (width 0.2) (layer "F.Cu") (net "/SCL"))
 (segment (start 236 85.8) (end 236.2 86) (width 0.2) (layer "F.Cu") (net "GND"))
 (segment (start 230.172 85.8) (end 236 85.8) (width 0.2) (layer "F.Cu") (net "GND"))
 (segment (start 229.16 84.788) (end 230.172 85.8) (width 0.2) (layer "F.Cu") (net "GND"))
 (segment (start 239.879 86) (end 252.014 73.865) (width 0.2) (layer "F.Cu") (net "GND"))
 (segment (start 236.2 86) (end 239.879 86) (width 0.2) (layer "F.Cu") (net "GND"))
 (segment (start 193.5 86) (end 189.11 81.61) (width 0.2) (layer "B.Cu") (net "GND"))
 (segment (start 236 101.88) (end 239.27 105.15) (width 0.2) (layer "B.Cu") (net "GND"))
 (segment (start 241.81 105.15) (end 242.96 104) (width 0.2) (layer "B.Cu") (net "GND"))
 (segment (start 252.014 73.865) (end 239.879 86) (width 0.2) (layer "B.Cu") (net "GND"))
 (segment (start 239.879 86) (end 236 86) (width 0.2) (layer "B.Cu") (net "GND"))
 (segment (start 189.11 81.61) (end 189.11 67.46) (width 0.2) (layer "B.Cu") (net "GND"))
 (segment (start 193.5 86) (end 236 86) (width 0.2) (layer "B.Cu") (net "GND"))
 (segment (start 195.61 106.46) (end 192.45 103.3) (width 0.2) (layer "B.Cu") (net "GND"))
 (segment (start 192.45 87.05) (end 193.5 86) (width 0.2) (layer "B.Cu") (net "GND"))
 (segment (start 236 86) (end 236 101.88) (width 0.2) (layer "B.Cu") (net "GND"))
 (segment (start 239.27 105.15) (end 241.81 105.15) (width 0.2) (layer "B.Cu") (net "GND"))
 (segment (start 192.45 103.3) (end 192.45 87.05) (width 0.2) (layer "B.Cu") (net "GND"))
 (segment (start 219.835 85.8) (end 198.78 85.8) (width 0.2) (layer "F.Cu") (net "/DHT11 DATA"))
 (segment (start 198.78 85.8) (end 193.5 91.08) (width 0.2) (layer "F.Cu") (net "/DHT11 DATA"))
 (segment (start 211.31 87.5) (end 218 87.5) (width 0.2) (layer "B.Cu") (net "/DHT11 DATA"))
 (segment (start 218 87.5) (end 219.1 86.4) (width 0.2) (layer "B.Cu") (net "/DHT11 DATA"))
 (segment (start 193.5 91.08) (end 207.73 91.08) (width 0.2) (layer "B.Cu") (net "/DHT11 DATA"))
 (segment (start 207.73 91.08) (end 211.31 87.5) (width 0.2) (layer "B.Cu") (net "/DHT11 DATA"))
 (segment (start 219.1 86.4) (end 220 86.4) (width 0.2) (layer "B.Cu") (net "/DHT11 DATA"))
 (segment (start 195.46 64.92) (end 204.008642 64.92) (width 0.2) (layer "F.Cu") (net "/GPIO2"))
 (segment (start 204.008642 64.92) (end 221.51 82.421358) (width 0.2) (layer "F.Cu") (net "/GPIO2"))
 (segment (start 221.51 82.421358) (end 221.51 86.665) (width 0.2) (layer "F.Cu") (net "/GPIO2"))
 (segment (start 221.51 86.665) (end 219.835 88.34) (width 0.2) (layer "F.Cu") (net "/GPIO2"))
 (segment (start 195.5 65) (end 195.5 64.96) (width 0.2) (layer "B.Cu") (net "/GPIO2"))
 (segment (start 195.46 64.92) (end 195.5 64.96) (width 0.2) (layer "B.Cu") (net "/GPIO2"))
 (segment (start 200.62 86.5) (end 194.55 92.57) (width 0.2) (layer "F.Cu") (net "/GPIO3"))
 (segment (start 219.835 90.88) (end 215.455 86.5) (width 0.2) (layer "F.Cu") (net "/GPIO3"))
 (segment (start 201.7 103.92) (end 201.96 103.92) (width 0.2) (layer "F.Cu") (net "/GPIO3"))
 (segment (start 192.45 92.57) (end 192.45 94.67) (width 0.2) (layer "F.Cu") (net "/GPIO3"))
 (segment (start 215.455 86.5) (end 200.62 86.5) (width 0.2) (layer "F.Cu") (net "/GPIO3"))
 (segment (start 192.45 94.67) (end 201.7 103.92) (width 0.2) (layer "F.Cu") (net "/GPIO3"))
 (segment (start 194.55 92.57) (end 192.45 92.57) (width 0.2) (layer "F.Cu") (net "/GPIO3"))
 (segment (start 201.96 103.92) (end 206.58 103.92) (width 0.2) (layer "B.Cu") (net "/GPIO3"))
 (segment (start 206.58 103.92) (end 220 90.5) (width 0.2) (layer "B.Cu") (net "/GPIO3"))
 (segment (start 226.5 82.368) (end 226.5 82.5) (width 0.2) (layer "F.Cu") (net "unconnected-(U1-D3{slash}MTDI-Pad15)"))
 (segment (start 226.62 82.248) (end 226.5 82.368) (width 0.2) (layer "F.Cu") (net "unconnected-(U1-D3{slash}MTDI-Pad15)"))
 (segment (start 193.5 88.54) (end 193.5 88.5) (width 0.2) (layer "F.Cu") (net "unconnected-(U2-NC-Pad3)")))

